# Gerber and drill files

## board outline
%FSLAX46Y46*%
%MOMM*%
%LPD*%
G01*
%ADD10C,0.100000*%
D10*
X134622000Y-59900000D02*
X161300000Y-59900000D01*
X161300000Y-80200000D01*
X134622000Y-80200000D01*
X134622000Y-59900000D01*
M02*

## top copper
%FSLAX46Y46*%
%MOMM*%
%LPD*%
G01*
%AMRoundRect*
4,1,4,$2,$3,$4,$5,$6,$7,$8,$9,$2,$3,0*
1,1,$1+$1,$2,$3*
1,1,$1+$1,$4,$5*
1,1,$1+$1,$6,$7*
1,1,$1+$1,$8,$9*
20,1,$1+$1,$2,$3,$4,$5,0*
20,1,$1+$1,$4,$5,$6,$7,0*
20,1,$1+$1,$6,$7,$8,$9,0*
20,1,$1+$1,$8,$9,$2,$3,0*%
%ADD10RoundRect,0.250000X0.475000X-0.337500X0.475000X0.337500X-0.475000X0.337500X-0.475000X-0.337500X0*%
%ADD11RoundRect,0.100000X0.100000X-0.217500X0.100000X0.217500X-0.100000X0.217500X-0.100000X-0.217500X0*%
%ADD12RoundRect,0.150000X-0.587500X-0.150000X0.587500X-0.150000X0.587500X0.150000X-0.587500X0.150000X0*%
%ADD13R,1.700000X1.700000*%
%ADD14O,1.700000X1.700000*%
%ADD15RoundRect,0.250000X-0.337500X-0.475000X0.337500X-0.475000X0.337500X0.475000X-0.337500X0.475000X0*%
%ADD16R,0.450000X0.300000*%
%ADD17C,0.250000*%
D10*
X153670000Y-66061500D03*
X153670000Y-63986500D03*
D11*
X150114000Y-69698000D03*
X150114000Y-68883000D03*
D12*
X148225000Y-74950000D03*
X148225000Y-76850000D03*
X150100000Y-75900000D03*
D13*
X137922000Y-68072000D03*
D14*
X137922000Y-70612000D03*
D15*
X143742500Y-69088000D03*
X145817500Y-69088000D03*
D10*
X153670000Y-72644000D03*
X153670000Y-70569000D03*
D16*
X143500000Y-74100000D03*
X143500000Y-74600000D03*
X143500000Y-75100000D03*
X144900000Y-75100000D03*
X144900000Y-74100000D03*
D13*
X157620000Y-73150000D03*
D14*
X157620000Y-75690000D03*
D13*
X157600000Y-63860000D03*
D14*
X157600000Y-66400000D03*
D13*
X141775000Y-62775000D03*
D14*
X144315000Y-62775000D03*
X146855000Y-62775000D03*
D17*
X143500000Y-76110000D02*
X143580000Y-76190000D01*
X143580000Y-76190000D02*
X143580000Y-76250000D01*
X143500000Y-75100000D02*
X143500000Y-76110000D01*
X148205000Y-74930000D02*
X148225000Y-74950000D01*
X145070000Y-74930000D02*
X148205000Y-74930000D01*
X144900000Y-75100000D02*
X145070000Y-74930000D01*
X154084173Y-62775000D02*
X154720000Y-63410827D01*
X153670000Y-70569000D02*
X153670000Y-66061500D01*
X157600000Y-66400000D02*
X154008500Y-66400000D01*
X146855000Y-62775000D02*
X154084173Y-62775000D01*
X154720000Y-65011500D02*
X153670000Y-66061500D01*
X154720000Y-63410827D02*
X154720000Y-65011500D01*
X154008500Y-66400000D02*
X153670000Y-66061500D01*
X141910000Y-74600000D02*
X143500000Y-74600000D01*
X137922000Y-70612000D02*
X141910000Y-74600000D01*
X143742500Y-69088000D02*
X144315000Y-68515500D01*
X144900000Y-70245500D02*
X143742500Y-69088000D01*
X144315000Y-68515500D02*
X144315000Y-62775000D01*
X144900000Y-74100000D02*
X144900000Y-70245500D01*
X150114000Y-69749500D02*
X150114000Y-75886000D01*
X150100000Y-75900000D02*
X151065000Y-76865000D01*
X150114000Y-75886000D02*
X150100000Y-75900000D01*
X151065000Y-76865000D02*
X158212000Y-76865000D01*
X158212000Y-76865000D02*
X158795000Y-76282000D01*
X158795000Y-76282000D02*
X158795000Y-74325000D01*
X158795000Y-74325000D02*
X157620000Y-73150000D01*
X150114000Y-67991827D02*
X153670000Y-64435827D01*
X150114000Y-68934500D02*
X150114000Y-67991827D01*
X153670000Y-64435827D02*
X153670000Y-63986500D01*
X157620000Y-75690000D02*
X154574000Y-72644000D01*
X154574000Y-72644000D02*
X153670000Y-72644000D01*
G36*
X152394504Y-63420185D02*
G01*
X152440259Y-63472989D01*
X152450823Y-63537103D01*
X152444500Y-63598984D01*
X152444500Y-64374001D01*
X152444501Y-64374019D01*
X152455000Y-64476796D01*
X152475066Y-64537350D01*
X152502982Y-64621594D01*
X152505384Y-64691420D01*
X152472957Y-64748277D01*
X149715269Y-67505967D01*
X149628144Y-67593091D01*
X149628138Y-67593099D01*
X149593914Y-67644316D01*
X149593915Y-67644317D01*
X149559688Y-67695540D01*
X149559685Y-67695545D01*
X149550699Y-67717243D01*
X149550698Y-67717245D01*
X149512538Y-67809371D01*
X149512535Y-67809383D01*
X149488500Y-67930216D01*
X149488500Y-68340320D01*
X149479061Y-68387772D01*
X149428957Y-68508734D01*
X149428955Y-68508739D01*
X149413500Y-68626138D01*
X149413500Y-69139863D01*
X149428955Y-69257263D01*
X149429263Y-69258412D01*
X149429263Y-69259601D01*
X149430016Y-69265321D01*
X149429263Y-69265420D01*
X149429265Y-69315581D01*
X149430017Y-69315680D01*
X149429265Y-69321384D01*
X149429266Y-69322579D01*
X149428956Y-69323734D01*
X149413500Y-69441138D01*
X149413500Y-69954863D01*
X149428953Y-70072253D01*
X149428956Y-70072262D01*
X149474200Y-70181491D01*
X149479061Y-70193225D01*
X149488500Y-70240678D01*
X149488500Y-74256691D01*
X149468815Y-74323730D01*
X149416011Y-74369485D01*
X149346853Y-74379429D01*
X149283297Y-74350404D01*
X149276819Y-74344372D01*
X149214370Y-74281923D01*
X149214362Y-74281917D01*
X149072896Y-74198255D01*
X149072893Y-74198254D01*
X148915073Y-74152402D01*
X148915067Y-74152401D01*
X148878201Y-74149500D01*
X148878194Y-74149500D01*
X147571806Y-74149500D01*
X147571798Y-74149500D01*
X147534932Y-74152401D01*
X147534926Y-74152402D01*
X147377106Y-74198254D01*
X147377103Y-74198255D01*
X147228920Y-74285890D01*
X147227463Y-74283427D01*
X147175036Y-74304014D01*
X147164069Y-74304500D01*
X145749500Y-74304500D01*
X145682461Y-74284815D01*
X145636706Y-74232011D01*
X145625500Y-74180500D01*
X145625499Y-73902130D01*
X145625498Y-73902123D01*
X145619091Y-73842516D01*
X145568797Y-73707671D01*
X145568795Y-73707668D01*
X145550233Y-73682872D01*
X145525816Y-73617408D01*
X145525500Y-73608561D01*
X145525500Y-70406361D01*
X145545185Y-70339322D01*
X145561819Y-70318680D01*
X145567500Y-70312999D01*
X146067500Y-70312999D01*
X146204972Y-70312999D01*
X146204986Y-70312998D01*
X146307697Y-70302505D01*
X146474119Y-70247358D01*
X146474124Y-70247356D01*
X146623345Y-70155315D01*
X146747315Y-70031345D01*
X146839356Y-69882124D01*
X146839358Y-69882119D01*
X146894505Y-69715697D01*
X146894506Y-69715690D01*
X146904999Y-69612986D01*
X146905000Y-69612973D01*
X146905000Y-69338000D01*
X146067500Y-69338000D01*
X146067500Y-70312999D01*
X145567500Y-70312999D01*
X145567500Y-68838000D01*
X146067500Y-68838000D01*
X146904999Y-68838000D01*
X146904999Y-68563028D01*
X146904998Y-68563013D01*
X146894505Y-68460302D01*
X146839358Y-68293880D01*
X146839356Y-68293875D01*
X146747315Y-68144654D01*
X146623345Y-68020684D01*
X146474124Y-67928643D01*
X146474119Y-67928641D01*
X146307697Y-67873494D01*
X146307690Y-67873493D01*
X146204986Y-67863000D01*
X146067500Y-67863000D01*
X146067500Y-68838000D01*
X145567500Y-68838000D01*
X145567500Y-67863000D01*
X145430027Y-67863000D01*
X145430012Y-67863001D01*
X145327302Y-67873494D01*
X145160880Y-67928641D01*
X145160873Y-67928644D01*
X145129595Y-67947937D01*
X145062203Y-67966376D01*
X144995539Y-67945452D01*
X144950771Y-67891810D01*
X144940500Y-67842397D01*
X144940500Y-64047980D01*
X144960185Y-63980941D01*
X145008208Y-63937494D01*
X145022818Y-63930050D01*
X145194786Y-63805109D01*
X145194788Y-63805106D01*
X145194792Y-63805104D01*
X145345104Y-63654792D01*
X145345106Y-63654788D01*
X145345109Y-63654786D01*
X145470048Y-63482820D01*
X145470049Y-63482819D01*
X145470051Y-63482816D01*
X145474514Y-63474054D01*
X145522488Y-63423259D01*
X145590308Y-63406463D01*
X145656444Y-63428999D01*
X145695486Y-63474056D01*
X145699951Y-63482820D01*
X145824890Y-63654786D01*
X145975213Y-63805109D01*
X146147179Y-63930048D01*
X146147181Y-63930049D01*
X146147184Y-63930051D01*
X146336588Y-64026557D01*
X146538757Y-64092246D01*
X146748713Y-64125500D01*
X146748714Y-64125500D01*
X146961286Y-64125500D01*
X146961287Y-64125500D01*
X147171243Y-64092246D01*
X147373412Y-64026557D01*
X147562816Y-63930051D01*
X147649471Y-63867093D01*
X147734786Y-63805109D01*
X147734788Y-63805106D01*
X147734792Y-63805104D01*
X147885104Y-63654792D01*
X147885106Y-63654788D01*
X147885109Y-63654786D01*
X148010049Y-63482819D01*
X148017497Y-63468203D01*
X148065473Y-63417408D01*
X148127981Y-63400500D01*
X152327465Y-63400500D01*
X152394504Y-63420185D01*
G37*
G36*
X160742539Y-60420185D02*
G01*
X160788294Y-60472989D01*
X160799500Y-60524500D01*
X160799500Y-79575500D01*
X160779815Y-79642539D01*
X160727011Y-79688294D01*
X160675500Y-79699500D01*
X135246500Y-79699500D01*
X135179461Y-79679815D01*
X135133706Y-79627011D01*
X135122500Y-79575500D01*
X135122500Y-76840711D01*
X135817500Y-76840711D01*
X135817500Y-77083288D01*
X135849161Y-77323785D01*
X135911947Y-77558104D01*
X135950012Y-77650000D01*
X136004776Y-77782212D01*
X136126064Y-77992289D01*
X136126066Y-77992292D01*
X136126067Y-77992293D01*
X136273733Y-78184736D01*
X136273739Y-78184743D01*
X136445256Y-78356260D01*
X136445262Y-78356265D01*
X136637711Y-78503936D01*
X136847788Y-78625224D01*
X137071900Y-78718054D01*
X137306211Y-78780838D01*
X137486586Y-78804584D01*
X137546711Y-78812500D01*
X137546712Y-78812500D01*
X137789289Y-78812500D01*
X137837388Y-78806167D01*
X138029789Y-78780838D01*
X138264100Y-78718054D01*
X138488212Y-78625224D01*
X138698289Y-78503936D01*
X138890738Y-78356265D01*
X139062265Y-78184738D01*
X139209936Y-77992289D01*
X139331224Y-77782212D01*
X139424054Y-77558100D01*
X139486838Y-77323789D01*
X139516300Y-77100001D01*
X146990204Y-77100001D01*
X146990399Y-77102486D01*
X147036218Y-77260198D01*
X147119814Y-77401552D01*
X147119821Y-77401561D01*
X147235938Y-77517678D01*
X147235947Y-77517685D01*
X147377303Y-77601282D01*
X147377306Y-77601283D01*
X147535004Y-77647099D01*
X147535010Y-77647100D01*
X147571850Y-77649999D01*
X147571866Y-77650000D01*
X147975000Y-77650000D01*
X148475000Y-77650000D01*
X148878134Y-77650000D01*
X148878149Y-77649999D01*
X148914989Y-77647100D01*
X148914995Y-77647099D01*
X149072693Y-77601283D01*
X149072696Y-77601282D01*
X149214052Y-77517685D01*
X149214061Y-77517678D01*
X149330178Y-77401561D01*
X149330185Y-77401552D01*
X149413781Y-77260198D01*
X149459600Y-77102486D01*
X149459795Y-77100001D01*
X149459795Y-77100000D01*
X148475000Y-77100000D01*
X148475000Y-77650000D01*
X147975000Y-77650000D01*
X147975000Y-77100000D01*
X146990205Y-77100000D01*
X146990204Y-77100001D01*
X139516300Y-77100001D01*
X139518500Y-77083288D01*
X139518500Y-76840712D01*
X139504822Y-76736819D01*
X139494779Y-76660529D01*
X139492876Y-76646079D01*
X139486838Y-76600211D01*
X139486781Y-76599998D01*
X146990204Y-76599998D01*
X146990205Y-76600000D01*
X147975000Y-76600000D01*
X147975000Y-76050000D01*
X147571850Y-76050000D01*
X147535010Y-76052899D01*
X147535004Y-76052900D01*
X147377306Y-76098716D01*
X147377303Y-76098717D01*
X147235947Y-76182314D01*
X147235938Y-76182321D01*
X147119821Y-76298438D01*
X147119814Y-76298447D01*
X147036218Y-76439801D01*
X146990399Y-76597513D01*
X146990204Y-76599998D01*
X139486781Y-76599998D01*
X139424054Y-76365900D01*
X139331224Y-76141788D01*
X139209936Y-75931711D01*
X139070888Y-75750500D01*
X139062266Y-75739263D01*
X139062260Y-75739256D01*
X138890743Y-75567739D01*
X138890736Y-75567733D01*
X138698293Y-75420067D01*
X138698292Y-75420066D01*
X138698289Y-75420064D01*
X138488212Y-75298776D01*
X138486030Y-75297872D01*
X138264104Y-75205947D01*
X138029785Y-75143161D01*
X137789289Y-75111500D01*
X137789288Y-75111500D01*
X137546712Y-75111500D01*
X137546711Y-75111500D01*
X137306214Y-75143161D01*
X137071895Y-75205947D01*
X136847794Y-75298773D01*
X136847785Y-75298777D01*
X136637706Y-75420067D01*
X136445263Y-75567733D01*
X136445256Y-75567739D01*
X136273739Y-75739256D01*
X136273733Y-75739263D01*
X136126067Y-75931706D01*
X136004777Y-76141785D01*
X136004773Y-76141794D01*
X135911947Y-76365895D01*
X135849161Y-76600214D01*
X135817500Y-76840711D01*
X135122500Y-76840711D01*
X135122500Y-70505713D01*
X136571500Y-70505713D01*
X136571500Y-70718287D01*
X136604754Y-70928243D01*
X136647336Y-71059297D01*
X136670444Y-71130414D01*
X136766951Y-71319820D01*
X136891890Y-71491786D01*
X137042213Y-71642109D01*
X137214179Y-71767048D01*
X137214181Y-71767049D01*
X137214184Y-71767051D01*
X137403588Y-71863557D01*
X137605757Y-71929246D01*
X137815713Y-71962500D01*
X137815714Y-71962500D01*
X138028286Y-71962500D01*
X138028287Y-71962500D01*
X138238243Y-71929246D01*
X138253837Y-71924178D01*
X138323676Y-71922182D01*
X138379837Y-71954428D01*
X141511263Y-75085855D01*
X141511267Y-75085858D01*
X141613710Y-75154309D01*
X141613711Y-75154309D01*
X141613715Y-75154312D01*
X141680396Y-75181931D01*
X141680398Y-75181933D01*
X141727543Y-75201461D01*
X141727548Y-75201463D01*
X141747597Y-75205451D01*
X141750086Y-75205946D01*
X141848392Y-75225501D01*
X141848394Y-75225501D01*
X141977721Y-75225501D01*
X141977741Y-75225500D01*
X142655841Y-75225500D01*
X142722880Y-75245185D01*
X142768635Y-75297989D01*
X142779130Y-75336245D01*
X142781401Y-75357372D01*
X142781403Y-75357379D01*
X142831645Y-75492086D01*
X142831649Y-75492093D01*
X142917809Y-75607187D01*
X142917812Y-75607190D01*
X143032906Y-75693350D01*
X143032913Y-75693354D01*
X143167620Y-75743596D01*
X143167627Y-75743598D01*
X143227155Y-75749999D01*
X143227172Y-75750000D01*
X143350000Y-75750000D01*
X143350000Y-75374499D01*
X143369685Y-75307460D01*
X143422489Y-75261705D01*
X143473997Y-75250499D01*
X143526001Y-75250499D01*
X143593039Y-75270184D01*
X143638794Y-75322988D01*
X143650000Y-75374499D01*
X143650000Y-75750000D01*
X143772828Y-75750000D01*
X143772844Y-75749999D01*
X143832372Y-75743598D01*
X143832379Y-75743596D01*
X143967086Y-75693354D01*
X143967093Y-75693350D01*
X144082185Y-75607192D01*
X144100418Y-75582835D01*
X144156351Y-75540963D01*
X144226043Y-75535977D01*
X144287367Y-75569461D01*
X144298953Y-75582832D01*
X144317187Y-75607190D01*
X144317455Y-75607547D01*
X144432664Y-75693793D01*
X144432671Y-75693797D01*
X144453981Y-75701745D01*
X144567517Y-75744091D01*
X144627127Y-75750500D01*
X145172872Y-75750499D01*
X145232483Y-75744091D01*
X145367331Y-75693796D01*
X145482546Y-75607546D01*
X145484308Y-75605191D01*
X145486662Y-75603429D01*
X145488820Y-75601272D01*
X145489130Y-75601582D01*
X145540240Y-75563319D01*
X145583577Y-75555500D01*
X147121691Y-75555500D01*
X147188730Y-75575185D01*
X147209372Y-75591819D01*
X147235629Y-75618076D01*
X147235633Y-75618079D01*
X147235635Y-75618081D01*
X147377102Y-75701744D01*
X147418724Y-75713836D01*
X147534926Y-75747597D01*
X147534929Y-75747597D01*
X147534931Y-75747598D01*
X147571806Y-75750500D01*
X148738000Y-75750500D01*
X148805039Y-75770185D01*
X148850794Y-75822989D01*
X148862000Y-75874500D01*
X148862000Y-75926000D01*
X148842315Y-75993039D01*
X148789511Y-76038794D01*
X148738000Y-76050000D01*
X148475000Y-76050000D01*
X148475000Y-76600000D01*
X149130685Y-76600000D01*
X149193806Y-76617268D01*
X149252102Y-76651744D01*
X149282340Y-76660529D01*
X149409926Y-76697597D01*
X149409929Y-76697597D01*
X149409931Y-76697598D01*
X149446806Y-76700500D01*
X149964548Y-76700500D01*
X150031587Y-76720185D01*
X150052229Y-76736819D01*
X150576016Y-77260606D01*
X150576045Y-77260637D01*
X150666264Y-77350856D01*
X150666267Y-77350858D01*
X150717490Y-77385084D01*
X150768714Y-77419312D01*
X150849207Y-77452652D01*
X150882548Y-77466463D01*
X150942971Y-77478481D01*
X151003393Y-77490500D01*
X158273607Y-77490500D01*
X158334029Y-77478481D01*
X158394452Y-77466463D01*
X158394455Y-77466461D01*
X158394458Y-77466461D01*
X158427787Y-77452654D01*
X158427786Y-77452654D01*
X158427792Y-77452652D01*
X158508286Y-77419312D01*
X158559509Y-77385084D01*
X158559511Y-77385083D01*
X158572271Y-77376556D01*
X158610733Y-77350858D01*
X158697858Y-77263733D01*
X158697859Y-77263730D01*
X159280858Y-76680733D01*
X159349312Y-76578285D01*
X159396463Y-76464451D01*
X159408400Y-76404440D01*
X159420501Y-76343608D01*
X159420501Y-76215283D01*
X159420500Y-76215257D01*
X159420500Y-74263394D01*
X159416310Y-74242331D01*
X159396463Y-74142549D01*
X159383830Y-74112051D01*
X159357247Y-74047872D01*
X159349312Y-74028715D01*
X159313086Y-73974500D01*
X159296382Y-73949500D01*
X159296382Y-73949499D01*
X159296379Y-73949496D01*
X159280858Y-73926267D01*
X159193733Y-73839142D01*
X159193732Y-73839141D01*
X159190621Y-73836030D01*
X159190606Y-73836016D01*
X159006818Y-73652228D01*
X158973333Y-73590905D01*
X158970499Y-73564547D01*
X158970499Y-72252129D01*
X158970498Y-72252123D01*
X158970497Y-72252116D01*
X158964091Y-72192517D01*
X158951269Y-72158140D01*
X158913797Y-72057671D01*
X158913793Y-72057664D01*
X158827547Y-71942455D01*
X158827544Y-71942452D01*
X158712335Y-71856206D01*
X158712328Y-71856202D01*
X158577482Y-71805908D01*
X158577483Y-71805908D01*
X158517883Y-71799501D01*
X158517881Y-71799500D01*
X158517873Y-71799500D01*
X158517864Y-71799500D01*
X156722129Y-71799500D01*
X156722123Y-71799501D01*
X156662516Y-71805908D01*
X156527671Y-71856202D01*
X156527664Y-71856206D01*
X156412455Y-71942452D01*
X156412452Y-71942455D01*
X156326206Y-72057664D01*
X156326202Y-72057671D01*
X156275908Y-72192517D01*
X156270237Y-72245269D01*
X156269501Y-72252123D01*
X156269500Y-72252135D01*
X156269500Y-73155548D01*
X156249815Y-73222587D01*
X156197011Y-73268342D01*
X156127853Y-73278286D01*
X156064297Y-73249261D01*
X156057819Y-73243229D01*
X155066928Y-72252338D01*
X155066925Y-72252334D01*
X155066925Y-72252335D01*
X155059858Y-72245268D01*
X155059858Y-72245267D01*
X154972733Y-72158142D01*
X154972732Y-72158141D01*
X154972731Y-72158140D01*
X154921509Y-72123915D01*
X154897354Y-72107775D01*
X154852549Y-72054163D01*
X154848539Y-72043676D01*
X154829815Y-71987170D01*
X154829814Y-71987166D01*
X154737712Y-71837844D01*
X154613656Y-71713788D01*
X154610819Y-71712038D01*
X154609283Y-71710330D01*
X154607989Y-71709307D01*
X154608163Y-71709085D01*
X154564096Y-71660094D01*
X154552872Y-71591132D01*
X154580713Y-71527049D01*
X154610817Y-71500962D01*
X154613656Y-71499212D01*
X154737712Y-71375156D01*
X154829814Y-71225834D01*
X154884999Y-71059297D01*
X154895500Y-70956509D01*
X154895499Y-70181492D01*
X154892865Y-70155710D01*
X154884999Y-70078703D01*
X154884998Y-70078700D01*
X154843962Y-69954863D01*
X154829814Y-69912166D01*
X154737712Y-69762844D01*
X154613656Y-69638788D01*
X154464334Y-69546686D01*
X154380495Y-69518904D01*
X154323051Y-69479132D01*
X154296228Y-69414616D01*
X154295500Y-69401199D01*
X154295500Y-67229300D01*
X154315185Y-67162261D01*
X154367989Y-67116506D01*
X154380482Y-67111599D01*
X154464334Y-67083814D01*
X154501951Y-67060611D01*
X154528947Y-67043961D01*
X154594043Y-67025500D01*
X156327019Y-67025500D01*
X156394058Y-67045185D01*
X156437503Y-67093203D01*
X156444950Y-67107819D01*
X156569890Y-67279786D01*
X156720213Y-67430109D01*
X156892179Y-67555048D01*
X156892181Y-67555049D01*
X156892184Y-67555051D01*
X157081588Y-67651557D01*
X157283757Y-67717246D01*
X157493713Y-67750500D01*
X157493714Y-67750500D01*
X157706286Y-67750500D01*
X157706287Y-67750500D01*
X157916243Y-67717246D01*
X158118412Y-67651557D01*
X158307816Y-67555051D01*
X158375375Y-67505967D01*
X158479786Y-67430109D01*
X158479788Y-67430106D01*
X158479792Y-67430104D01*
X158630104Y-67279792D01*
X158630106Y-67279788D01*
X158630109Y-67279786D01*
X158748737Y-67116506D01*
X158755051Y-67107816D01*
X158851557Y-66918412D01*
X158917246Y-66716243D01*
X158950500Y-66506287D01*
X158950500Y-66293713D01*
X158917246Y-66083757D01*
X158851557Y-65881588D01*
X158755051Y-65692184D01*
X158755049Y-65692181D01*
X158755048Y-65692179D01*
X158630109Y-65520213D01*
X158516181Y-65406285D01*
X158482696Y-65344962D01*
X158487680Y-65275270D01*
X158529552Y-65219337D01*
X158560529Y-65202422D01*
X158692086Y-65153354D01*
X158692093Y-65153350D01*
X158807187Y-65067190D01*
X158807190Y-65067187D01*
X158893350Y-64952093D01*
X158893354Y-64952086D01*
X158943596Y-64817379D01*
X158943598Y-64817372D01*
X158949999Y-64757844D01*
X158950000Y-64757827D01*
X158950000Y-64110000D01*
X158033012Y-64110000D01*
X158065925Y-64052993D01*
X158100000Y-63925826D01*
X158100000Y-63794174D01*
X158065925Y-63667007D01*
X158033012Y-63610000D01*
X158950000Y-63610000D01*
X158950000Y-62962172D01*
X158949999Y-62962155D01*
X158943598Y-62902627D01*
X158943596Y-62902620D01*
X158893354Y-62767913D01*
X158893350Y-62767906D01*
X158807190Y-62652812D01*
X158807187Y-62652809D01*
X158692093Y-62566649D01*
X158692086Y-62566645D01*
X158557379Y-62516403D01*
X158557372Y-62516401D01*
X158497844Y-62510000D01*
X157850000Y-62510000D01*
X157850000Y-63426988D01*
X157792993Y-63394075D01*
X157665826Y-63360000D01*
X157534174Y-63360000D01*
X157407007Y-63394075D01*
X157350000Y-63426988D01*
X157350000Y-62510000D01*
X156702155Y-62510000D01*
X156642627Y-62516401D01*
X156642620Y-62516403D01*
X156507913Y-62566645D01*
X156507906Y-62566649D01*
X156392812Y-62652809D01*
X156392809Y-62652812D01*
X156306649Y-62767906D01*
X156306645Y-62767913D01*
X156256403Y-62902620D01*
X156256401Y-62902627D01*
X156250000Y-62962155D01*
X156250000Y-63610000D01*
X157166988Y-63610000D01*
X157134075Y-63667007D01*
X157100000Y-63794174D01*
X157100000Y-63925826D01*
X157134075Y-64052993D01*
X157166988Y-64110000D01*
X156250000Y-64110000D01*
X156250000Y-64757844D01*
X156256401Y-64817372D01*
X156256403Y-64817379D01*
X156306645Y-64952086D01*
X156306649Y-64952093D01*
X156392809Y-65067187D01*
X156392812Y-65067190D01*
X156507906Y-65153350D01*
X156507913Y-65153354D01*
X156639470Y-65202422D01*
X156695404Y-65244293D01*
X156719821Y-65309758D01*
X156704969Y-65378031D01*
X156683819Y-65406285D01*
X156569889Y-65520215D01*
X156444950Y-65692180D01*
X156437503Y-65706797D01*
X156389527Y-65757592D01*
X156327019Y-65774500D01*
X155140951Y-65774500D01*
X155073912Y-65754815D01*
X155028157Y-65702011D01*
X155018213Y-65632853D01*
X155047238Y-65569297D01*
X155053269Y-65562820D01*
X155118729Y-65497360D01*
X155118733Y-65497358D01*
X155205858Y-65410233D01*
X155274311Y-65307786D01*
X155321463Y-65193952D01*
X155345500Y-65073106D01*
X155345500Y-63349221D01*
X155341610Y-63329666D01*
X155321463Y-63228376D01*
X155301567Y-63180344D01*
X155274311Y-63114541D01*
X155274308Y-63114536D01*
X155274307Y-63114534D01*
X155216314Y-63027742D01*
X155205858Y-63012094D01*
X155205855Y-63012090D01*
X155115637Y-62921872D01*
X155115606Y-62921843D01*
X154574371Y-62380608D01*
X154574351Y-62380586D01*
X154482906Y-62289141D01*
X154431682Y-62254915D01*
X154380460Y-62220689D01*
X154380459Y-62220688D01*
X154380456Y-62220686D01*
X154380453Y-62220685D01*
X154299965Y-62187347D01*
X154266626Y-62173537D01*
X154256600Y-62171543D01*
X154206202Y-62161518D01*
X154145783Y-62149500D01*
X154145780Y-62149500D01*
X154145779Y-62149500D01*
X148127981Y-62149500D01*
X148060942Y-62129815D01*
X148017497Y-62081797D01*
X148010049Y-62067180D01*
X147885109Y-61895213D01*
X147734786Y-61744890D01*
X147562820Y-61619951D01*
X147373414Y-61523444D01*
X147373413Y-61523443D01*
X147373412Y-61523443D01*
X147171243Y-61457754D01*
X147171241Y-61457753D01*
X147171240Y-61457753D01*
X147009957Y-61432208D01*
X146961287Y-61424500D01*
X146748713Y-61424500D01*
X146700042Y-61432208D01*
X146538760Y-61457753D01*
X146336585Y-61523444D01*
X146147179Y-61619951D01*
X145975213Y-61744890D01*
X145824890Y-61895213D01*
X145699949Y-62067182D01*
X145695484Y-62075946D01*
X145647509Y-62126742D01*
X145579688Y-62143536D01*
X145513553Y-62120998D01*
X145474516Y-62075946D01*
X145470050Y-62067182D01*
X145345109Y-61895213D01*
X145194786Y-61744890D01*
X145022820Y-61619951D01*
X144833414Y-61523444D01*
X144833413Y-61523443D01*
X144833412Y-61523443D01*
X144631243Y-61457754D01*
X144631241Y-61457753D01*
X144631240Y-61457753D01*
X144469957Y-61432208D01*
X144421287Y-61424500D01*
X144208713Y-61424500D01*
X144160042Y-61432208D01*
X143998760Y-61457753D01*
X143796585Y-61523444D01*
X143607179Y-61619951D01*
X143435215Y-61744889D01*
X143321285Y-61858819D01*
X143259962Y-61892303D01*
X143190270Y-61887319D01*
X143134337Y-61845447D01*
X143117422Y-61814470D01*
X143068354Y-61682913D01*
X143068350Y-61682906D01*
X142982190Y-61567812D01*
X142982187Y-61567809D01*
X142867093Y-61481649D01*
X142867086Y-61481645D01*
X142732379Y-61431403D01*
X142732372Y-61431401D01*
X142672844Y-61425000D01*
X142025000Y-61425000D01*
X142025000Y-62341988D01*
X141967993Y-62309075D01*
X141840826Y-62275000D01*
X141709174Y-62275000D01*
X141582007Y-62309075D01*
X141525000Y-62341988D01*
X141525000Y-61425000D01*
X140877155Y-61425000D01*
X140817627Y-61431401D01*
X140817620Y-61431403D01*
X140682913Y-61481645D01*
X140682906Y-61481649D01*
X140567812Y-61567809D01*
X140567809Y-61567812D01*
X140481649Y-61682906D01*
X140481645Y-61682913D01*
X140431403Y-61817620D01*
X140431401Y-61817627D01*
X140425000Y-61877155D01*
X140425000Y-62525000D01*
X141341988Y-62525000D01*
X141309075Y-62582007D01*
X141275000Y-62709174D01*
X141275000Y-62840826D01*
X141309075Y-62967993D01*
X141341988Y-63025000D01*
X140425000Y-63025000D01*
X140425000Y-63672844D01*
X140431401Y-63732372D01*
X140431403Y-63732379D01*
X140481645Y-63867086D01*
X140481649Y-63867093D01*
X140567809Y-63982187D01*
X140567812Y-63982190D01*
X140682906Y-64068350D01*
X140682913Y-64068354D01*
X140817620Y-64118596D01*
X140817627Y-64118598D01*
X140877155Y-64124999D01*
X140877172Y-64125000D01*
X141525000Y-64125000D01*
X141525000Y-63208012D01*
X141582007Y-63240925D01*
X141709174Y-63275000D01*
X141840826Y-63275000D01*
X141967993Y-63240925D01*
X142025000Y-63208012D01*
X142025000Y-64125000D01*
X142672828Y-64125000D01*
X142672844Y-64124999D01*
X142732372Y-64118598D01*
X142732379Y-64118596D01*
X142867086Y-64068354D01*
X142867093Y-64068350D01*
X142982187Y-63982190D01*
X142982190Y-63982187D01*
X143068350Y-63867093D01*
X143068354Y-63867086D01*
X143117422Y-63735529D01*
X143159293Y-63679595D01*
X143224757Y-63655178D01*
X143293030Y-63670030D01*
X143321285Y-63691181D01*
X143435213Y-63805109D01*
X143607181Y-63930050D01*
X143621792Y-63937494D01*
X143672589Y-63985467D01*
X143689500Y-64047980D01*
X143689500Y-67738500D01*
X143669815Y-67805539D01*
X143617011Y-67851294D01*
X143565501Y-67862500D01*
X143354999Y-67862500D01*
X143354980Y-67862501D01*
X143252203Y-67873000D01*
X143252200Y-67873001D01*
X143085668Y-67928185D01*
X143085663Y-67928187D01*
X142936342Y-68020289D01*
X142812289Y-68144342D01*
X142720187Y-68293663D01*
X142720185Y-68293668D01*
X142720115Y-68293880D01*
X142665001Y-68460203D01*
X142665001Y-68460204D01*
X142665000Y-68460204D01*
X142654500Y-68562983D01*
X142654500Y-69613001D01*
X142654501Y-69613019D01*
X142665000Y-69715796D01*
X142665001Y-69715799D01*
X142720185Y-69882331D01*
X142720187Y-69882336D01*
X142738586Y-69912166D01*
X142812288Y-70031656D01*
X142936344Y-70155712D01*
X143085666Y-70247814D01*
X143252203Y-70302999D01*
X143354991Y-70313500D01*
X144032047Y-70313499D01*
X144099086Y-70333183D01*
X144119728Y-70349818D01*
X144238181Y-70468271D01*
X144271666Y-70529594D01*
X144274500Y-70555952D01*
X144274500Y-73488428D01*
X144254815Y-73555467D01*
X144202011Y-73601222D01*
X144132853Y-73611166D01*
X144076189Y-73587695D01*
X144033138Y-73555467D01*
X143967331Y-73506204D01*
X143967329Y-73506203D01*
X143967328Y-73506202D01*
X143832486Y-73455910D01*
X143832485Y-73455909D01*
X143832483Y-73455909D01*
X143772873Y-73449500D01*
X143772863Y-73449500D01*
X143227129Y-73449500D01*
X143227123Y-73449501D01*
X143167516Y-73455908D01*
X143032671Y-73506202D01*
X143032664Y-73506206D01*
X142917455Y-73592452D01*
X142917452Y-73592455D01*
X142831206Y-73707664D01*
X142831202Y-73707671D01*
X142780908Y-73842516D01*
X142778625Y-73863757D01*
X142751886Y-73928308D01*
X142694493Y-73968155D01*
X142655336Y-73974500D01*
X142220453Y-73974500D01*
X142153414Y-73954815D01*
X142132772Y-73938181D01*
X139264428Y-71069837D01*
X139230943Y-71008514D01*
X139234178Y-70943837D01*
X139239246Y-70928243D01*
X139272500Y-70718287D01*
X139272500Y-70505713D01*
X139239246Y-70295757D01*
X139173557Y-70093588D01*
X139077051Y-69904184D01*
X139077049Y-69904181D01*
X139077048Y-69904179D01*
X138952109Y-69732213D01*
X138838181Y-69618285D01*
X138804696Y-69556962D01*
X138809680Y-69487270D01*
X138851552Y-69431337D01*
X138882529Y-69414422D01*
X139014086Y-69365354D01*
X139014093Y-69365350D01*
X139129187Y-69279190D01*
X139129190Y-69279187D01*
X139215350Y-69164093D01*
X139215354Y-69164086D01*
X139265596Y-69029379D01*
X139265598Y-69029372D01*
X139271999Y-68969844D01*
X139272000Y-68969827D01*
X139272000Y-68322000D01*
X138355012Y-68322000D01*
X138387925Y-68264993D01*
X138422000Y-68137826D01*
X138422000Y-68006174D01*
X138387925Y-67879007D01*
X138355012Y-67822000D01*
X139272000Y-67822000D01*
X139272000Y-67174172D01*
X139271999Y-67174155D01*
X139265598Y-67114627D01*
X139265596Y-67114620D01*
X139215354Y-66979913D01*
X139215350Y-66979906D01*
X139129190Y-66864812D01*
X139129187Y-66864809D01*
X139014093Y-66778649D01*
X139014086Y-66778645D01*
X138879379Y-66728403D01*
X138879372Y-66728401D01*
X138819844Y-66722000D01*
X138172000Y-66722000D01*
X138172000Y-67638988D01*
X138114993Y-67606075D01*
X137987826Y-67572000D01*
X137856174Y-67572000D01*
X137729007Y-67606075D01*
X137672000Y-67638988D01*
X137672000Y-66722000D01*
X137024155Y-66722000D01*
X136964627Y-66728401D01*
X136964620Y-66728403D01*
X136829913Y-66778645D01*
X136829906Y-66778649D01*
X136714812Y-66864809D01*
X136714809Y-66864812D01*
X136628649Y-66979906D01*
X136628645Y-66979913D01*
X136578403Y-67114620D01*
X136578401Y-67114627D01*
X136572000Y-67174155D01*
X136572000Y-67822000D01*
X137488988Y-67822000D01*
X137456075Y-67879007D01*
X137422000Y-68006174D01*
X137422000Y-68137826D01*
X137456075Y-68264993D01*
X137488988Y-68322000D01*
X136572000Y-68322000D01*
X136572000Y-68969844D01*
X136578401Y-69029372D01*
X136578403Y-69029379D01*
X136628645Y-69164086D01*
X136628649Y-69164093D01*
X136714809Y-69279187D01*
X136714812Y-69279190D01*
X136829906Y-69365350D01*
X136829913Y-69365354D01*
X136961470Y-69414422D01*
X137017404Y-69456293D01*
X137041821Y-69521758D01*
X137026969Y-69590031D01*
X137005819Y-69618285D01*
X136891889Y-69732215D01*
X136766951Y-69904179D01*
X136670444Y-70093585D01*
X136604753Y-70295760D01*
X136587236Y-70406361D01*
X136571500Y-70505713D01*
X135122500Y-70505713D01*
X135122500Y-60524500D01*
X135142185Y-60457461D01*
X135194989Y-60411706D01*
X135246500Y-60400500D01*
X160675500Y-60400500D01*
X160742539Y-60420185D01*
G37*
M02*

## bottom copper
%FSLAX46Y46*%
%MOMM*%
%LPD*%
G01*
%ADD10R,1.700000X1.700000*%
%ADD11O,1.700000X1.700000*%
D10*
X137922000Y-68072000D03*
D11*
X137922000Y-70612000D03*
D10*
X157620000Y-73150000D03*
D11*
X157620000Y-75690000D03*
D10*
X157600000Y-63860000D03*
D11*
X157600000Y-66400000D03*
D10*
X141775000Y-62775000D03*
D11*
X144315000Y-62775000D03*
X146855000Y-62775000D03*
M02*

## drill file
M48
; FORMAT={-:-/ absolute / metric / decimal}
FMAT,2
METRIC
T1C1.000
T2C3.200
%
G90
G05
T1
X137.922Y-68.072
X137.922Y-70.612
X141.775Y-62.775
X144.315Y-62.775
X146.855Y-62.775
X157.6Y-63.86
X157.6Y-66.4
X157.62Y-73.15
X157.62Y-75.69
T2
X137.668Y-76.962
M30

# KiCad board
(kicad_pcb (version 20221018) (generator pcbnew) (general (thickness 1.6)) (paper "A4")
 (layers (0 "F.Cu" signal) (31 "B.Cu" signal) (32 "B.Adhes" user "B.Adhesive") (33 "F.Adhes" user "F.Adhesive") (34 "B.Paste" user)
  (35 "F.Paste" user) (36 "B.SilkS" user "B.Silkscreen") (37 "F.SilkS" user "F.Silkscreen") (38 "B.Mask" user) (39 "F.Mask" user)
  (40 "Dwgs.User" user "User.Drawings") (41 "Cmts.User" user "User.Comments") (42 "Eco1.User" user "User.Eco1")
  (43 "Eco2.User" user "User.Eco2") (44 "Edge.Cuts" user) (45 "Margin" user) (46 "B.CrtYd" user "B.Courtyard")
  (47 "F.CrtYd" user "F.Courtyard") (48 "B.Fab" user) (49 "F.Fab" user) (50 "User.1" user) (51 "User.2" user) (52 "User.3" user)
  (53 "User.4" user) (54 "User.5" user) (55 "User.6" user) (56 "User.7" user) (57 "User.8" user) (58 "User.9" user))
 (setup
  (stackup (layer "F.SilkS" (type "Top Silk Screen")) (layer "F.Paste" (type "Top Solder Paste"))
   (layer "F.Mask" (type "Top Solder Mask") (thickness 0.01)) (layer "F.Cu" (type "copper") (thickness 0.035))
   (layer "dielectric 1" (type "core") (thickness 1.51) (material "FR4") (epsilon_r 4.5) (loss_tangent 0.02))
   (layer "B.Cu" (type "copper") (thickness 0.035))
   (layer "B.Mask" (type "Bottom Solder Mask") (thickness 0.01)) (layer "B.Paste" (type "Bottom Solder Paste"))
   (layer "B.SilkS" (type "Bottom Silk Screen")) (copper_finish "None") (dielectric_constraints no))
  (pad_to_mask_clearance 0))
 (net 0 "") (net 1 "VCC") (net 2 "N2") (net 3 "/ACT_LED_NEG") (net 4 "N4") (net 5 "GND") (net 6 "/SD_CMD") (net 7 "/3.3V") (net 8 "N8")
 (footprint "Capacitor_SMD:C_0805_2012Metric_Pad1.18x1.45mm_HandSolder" (layer "F.Cu") (at 153.67 65.024 90)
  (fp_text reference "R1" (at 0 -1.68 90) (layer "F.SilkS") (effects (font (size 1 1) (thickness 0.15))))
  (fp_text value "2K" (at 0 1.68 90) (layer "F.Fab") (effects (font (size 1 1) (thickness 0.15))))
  (pad "1" smd roundrect (at -1.0375 0 90) (size 1.175 1.45) (layers "F.Cu" "F.Paste" "F.Mask") (roundrect_rratio 0.2127659574)
   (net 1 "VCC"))
  (pad "2" smd roundrect (at 1.0375 0 90) (size 1.175 1.45) (layers "F.Cu" "F.Paste" "F.Mask") (roundrect_rratio 0.2127659574) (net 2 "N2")))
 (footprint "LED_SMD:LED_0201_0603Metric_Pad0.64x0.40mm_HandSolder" (layer "F.Cu") (at 150.114 69.2905 90)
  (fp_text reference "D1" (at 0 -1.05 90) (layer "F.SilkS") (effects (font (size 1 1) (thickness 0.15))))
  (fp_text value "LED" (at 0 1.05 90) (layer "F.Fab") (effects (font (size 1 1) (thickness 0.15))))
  (pad "" smd roundrect (at -0.4325 0 90) (size 0.458 0.36) (layers "F.Paste") (roundrect_rratio 0.25))
  (pad "" smd roundrect (at 0.4325 0 90) (size 0.458 0.36) (layers "F.Paste") (roundrect_rratio 0.25))
  (pad "1" smd roundrect (at -0.4075 0 90) (size 0.635 0.4) (layers "F.Cu" "F.Mask") (roundrect_rratio 0.25) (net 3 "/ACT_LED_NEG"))
  (pad "2" smd roundrect (at 0.4075 0 90) (size 0.635 0.4) (layers "F.Cu" "F.Mask") (roundrect_rratio 0.25) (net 2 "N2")))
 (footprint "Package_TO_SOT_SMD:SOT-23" (layer "F.Cu") (at 149.1625 75.9)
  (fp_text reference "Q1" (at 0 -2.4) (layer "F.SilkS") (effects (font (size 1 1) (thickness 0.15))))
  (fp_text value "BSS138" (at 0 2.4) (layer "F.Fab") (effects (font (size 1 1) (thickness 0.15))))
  (pad "1" smd roundrect (at -0.9375 -0.95) (size 1.475 0.6) (layers "F.Cu" "F.Paste" "F.Mask") (roundrect_rratio 0.25) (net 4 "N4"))
  (pad "2" smd roundrect (at -0.9375 0.95) (size 1.475 0.6) (layers "F.Cu" "F.Paste" "F.Mask") (roundrect_rratio 0.25) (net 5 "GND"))
  (pad "3" smd roundrect (at 0.9375 0) (size 1.475 0.6) (layers "F.Cu" "F.Paste" "F.Mask") (roundrect_rratio 0.25) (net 3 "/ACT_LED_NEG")))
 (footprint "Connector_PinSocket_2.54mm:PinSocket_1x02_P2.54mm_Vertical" (layer "F.Cu") (at 137.922 68.072)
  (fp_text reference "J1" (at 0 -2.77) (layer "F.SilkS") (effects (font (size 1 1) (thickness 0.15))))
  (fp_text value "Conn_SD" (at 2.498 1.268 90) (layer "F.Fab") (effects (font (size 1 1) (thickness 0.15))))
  (pad "1" thru_hole rect (at 0 0) (size 1.7 1.7) (drill 1) (layers "*.Cu" "*.Mask") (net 5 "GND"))
  (pad "2" thru_hole oval (at 0 2.54) (size 1.7 1.7) (drill 1) (layers "*.Cu" "*.Mask") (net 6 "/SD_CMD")))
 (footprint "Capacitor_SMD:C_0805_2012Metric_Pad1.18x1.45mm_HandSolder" (layer "F.Cu") (at 144.78 69.088)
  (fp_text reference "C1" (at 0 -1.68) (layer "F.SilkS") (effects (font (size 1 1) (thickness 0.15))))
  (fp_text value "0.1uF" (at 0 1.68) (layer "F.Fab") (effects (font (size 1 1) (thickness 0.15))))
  (pad "1" smd roundrect (at -1.0375 0) (size 1.175 1.45) (layers "F.Cu" "F.Paste" "F.Mask") (roundrect_rratio 0.2127659574) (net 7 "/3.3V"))
  (pad "2" smd roundrect (at 1.0375 0) (size 1.175 1.45) (layers "F.Cu" "F.Paste" "F.Mask") (roundrect_rratio 0.2127659574) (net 5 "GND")))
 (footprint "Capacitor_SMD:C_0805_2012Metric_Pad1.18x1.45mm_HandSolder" (layer "F.Cu") (at 153.67 71.6065 90)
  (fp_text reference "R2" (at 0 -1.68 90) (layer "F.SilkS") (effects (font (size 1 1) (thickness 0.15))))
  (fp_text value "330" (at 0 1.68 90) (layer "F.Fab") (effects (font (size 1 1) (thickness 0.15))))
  (pad "1" smd roundrect (at -1.0375 0 90) (size 1.175 1.45) (layers "F.Cu" "F.Paste" "F.Mask") (roundrect_rratio 0.2127659574) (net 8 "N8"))
  (pad "2" smd roundrect (at 1.0375 0 90) (size 1.175 1.45) (layers "F.Cu" "F.Paste" "F.Mask") (roundrect_rratio 0.2127659574) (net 1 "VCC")))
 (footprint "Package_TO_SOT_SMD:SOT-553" (layer "F.Cu") (at 144.2 74.6)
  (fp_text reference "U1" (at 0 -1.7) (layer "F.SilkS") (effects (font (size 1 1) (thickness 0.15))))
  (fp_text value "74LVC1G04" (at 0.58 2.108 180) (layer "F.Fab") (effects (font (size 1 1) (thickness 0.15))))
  (pad "1" smd rect (at -0.7 -0.5) (size 0.45 0.3) (layers "F.Cu" "F.Paste" "F.Mask"))
  (pad "2" smd rect (at -0.7 0) (size 0.45 0.3) (layers "F.Cu" "F.Paste" "F.Mask") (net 6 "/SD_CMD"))
  (pad "3" smd rect (at -0.7 0.5) (size 0.45 0.3) (layers "F.Cu" "F.Paste" "F.Mask") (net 5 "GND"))
  (pad "4" smd rect (at 0.7 0.5) (size 0.45 0.3) (layers "F.Cu" "F.Paste" "F.Mask") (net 4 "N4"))
  (pad "5" smd rect (at 0.7 -0.5) (size 0.45 0.3) (layers "F.Cu" "F.Paste" "F.Mask") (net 7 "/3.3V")))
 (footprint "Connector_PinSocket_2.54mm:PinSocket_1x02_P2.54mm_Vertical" (layer "F.Cu") (at 157.62 73.15)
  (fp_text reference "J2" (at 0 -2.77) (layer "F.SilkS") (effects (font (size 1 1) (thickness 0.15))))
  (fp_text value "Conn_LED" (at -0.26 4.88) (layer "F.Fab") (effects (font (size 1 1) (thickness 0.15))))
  (pad "1" thru_hole rect (at 0 0) (size 1.7 1.7) (drill 1) (layers "*.Cu" "*.Mask") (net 3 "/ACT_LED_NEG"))
  (pad "2" thru_hole oval (at 0 2.54) (size 1.7 1.7) (drill 1) (layers "*.Cu" "*.Mask") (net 8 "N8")))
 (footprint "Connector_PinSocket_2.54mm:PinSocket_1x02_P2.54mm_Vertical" (layer "F.Cu") (at 157.6 63.86)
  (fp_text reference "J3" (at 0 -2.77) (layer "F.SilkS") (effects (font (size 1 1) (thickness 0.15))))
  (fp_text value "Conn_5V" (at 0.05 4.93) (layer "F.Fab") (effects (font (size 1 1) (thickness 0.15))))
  (pad "1" thru_hole rect (at 0 0) (size 1.7 1.7) (drill 1) (layers "*.Cu" "*.Mask") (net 5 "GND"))
  (pad "2" thru_hole oval (at 0 2.54) (size 1.7 1.7) (drill 1) (layers "*.Cu" "*.Mask") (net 1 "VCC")))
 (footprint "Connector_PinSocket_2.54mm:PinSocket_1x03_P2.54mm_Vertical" (layer "F.Cu") (at 141.775 62.775 90)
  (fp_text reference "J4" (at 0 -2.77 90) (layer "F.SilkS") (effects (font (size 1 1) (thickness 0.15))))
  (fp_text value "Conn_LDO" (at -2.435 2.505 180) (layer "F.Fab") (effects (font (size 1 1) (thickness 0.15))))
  (pad "1" thru_hole rect (at 0 0 90) (size 1.7 1.7) (drill 1) (layers "*.Cu" "*.Mask") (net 5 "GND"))
  (pad "2" thru_hole oval (at 0 2.54 90) (size 1.7 1.7) (drill 1) (layers "*.Cu" "*.Mask") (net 7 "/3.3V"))
  (pad "3" thru_hole oval (at 0 5.08 90) (size 1.7 1.7) (drill 1) (layers "*.Cu" "*.Mask") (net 1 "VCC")))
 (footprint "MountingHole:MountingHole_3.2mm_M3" (layer "F.Cu") (at 137.668 76.962)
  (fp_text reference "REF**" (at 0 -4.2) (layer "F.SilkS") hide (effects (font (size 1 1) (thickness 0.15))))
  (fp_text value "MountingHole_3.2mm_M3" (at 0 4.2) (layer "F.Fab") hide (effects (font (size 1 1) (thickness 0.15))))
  (pad "" np_thru_hole circle (at 0 0) (size 3.2 3.2) (drill 3.2) (layers "*.Cu" "*.Mask")))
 (gr_rect (start 134.622 59.9) (end 161.3 80.2) (stroke (width 0.1) (type default)) (fill none) (layer "Edge.Cuts"))
 (segment (start 143.5 76.11) (end 143.58 76.19) (width 0.25) (layer "F.Cu") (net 5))
 (segment (start 143.58 76.19) (end 143.58 76.25) (width 0.25) (layer "F.Cu") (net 5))
 (segment (start 143.5 75.1) (end 143.5 76.11) (width 0.25) (layer "F.Cu") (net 5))
 (segment (start 148.205 74.93) (end 148.225 74.95) (width 0.25) (layer "F.Cu") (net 4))
 (segment (start 145.07 74.93) (end 148.205 74.93) (width 0.25) (layer "F.Cu") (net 4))
 (segment (start 144.9 75.1) (end 145.07 74.93) (width 0.25) (layer "F.Cu") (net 4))
 (segment (start 154.084173 62.775) (end 154.72 63.410827) (width 0.25) (layer "F.Cu") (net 1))
 (segment (start 153.67 70.569) (end 153.67 66.0615) (width 0.25) (layer "F.Cu") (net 1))
 (segment (start 157.6 66.4) (end 154.0085 66.4) (width 0.25) (layer "F.Cu") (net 1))
 (segment (start 146.855 62.775) (end 154.084173 62.775) (width 0.25) (layer "F.Cu") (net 1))
 (segment (start 154.72 65.0115) (end 153.67 66.0615) (width 0.25) (layer "F.Cu") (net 1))
 (segment (start 154.72 63.410827) (end 154.72 65.0115) (width 0.25) (layer "F.Cu") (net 1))
 (segment (start 154.0085 66.4) (end 153.67 66.0615) (width 0.25) (layer "F.Cu") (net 1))
 (segment (start 141.91 74.6) (end 143.5 74.6) (width 0.25) (layer "F.Cu") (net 6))
 (segment (start 137.922 70.612) (end 141.91 74.6) (width 0.25) (layer "F.Cu") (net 6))
 (segment (start 143.7425 69.088) (end 144.315 68.5155) (width 0.25) (layer "F.Cu") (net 7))
 (segment (start 144.9 70.2455) (end 143.7425 69.088) (width 0.25) (layer "F.Cu") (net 7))
 (segment (start 144.315 68.5155) (end 144.315 62.775) (width 0.25) (layer "F.Cu") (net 7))
 (segment (start 144.9 74.1) (end 144.9 70.2455) (width 0.25) (layer "F.Cu") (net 7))
 (segment (start 150.114 69.7495) (end 150.114 75.886) (width 0.25) (layer "F.Cu") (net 3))
 (segment (start 150.1 75.9) (end 151.065 76.865) (width 0.25) (layer "F.Cu") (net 3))
 (segment (start 150.114 75.886) (end 150.1 75.9) (width 0.25) (layer "F.Cu") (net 3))
 (segment (start 151.065 76.865) (end 158.212 76.865) (width 0.25) (layer "F.Cu") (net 3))
 (segment (start 158.212 76.865) (end 158.795 76.282) (width 0.25) (layer "F.Cu") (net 3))
 (segment (start 158.795 76.282) (end 158.795 74.325) (width 0.25) (layer "F.Cu") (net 3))
 (segment (start 158.795 74.325) (end 157.62 73.15) (width 0.25) (layer "F.Cu") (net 3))
 (segment (start 150.114 67.991827) (end 153.67 64.435827) (width 0.25) (layer "F.Cu") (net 2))
 (segment (start 150.114 68.9345) (end 150.114 67.991827) (width 0.25) (layer "F.Cu") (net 2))
 (segment (start 153.67 64.435827) (end 153.67 63.9865) (width 0.25) (layer "F.Cu") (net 2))
 (segment (start 157.62 75.69) (end 154.574 72.644) (width 0.25) (layer "F.Cu") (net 8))
 (segment (start 154.574 72.644) (end 153.67 72.644) (width 0.25) (layer "F.Cu") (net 8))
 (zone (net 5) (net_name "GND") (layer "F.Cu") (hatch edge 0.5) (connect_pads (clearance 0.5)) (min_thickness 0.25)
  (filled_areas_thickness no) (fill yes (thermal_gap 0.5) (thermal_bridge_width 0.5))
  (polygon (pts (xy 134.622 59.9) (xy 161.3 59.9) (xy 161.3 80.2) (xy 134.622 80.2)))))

